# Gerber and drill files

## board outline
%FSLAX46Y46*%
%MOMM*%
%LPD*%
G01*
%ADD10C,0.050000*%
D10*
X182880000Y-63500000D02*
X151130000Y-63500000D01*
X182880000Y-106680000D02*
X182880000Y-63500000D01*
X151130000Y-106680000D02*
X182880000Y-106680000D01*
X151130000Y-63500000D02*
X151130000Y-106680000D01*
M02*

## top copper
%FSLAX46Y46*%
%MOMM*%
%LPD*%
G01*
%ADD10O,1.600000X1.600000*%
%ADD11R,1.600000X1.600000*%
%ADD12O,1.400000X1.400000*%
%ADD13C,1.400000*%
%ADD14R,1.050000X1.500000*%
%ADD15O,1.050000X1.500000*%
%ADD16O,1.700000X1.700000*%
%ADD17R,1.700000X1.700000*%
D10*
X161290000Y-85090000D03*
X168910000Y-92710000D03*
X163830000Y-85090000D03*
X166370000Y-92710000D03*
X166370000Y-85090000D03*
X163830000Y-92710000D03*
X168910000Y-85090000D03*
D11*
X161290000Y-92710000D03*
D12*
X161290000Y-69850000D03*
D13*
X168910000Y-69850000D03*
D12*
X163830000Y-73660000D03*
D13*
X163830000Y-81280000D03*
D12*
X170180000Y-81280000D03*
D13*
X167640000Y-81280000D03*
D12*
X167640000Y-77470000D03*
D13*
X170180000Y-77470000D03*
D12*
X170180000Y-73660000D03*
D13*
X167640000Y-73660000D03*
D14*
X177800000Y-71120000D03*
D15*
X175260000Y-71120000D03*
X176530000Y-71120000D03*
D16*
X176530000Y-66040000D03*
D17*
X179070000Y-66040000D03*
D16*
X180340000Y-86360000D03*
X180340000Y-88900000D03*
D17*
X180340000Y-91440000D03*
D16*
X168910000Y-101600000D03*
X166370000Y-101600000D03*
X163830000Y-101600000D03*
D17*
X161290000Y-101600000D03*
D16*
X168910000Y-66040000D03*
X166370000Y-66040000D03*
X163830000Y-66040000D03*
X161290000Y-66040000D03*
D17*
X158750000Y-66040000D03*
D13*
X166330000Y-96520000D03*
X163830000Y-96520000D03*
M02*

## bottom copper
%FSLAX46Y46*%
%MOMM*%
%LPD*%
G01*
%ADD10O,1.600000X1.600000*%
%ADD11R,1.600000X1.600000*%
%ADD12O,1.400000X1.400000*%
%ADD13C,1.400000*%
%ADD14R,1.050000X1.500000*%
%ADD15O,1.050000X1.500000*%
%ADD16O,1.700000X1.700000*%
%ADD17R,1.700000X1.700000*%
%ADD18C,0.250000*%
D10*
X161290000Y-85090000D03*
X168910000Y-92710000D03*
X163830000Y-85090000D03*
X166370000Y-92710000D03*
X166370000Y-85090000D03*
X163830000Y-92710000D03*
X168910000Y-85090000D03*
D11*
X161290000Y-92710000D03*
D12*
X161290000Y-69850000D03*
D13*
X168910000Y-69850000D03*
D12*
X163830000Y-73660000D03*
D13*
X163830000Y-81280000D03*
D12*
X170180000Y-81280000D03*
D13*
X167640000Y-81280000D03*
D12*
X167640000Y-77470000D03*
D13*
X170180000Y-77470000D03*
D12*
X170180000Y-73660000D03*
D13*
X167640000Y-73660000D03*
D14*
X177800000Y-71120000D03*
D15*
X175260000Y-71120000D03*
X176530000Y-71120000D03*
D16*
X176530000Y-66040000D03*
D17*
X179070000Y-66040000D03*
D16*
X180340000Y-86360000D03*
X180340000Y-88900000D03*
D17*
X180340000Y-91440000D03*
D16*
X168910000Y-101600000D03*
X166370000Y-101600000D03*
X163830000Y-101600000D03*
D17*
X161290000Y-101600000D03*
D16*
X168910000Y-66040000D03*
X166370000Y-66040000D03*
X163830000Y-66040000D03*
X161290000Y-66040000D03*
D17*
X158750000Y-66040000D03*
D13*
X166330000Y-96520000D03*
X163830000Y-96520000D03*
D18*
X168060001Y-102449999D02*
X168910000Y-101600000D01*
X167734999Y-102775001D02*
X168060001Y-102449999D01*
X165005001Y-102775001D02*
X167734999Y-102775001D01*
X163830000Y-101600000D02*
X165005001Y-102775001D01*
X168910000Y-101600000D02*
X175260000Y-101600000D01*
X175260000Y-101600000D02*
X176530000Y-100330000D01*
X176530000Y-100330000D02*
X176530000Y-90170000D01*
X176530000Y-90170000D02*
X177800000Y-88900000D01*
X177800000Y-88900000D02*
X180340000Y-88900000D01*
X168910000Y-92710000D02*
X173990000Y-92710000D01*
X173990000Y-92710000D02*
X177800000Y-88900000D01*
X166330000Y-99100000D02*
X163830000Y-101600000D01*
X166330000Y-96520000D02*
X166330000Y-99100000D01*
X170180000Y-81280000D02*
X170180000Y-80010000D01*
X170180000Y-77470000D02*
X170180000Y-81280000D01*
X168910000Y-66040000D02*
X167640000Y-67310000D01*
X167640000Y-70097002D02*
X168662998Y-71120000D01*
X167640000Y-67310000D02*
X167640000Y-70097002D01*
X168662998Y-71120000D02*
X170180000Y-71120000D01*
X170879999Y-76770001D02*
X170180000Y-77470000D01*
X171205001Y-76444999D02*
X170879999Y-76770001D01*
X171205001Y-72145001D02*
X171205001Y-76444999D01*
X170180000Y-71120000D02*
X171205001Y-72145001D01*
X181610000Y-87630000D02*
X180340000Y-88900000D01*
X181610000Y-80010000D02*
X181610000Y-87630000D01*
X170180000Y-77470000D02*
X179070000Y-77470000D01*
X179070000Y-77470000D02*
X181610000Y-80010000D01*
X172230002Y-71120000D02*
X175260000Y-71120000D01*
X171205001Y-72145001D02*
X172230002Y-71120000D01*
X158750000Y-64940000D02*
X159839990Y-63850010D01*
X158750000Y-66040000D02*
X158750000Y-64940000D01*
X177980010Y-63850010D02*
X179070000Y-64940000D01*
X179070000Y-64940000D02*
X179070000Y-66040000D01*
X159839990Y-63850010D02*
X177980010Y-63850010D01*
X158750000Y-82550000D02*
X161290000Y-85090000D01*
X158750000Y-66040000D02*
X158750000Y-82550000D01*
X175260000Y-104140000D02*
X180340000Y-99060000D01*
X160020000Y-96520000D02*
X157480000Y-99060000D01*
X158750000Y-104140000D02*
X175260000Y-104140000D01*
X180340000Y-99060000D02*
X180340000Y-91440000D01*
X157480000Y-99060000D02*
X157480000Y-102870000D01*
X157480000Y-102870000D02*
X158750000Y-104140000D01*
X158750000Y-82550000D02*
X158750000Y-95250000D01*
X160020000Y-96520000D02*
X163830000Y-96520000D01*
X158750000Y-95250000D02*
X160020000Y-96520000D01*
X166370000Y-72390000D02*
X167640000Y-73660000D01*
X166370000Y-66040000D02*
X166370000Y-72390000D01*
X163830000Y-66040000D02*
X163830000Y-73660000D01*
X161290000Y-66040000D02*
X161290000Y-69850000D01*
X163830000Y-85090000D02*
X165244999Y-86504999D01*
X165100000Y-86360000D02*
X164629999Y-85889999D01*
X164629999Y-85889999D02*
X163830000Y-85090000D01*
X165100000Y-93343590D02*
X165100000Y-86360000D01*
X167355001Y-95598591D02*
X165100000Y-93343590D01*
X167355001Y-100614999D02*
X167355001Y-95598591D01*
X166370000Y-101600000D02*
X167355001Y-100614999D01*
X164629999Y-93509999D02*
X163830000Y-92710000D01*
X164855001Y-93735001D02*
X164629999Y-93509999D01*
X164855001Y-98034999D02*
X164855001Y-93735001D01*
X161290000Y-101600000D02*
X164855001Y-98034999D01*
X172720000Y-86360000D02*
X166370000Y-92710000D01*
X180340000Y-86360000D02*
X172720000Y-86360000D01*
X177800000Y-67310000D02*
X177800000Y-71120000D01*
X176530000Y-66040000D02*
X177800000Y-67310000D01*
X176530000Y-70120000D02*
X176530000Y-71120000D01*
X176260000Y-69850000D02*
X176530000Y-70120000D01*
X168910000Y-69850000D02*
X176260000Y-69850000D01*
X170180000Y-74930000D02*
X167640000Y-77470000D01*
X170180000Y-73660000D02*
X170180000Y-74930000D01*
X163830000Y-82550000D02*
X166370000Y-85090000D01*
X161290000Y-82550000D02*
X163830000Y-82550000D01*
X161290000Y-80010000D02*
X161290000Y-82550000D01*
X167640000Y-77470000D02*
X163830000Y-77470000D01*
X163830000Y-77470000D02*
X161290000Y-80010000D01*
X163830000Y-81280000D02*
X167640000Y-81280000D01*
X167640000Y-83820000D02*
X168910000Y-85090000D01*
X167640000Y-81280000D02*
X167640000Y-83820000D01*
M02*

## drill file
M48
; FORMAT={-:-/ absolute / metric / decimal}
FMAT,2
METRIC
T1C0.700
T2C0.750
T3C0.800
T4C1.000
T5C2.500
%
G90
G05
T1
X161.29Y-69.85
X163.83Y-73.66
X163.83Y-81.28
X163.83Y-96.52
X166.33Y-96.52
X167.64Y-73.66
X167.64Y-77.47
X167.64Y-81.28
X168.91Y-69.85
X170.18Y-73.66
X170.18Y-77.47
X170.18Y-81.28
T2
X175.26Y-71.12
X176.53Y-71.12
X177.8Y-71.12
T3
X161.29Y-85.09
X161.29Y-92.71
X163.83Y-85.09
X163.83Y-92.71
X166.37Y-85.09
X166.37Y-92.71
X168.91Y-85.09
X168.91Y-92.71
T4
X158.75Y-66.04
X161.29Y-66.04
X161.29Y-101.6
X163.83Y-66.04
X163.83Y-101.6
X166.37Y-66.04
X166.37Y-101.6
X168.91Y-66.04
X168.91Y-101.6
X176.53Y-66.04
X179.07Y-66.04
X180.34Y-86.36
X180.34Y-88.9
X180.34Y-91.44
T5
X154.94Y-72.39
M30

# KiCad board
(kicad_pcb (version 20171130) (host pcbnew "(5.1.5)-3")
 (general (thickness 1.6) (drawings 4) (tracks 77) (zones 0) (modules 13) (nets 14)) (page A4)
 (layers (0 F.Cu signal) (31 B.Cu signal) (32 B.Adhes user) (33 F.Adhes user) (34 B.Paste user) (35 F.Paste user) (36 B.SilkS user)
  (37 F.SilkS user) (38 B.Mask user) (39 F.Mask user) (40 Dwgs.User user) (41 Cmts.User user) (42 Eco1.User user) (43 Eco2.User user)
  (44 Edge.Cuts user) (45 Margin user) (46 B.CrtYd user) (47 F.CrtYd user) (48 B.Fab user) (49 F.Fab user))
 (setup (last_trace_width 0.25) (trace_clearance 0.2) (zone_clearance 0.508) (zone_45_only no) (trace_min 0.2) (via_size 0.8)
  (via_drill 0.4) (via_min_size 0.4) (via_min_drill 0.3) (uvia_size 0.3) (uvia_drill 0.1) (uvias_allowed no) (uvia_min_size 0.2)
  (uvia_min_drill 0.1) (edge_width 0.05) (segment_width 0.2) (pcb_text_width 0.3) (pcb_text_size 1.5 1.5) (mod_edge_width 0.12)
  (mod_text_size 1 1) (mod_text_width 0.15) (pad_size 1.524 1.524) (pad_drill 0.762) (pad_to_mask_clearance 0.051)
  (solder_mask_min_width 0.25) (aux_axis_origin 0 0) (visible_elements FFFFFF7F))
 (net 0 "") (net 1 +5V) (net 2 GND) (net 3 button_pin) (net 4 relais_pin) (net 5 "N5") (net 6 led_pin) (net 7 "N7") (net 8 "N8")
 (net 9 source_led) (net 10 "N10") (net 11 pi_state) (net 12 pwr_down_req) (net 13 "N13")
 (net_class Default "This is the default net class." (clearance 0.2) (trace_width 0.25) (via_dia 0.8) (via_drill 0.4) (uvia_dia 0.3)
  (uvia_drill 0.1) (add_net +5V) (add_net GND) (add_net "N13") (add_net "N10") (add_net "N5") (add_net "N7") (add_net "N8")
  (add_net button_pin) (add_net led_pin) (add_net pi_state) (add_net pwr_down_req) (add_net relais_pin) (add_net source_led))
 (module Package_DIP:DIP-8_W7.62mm (layer F.Cu) (at 161.29 92.71 90)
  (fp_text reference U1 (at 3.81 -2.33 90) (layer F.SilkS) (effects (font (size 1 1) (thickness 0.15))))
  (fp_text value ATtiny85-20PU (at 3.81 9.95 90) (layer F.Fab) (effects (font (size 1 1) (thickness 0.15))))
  (pad 8 thru_hole oval (at 7.62 0 90) (size 1.6 1.6) (drill 0.8) (layers *.Cu *.Mask) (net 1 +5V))
  (pad 4 thru_hole oval (at 0 7.62 90) (size 1.6 1.6) (drill 0.8) (layers *.Cu *.Mask) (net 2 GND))
  (pad 7 thru_hole oval (at 7.62 2.54 90) (size 1.6 1.6) (drill 0.8) (layers *.Cu *.Mask) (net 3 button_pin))
  (pad 3 thru_hole oval (at 0 5.08 90) (size 1.6 1.6) (drill 0.8) (layers *.Cu *.Mask) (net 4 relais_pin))
  (pad 6 thru_hole oval (at 7.62 5.08 90) (size 1.6 1.6) (drill 0.8) (layers *.Cu *.Mask) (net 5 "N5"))
  (pad 2 thru_hole oval (at 0 2.54 90) (size 1.6 1.6) (drill 0.8) (layers *.Cu *.Mask) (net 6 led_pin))
  (pad 5 thru_hole oval (at 7.62 7.62 90) (size 1.6 1.6) (drill 0.8) (layers *.Cu *.Mask) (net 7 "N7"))
  (pad 1 thru_hole rect (at 0 0 90) (size 1.6 1.6) (drill 0.8) (layers *.Cu *.Mask) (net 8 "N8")))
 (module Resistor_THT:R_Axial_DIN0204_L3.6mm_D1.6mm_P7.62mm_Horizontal (layer F.Cu) (at 168.91 69.85 180)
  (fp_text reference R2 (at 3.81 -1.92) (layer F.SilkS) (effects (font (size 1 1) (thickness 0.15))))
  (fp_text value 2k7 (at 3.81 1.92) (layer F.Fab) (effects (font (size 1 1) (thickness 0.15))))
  (pad 2 thru_hole oval (at 7.62 0 180) (size 1.4 1.4) (drill 0.7) (layers *.Cu *.Mask) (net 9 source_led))
  (pad 1 thru_hole circle (at 0 0 180) (size 1.4 1.4) (drill 0.7) (layers *.Cu *.Mask) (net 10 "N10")))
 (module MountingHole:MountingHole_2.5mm (layer F.Cu) (at 154.94 72.39)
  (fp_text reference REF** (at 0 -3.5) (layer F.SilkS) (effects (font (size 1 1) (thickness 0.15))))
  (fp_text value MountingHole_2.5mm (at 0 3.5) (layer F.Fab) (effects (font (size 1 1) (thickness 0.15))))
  (pad 1 np_thru_hole circle (at 0 0) (size 2.5 2.5) (drill 2.5) (layers *.Cu *.Mask)))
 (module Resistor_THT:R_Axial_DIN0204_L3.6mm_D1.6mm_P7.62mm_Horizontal (layer F.Cu) (at 163.83 81.28 90)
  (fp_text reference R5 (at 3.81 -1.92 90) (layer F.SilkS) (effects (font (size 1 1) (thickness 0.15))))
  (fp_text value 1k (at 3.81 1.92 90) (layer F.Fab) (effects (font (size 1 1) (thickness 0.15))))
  (pad 2 thru_hole oval (at 7.62 0 90) (size 1.4 1.4) (drill 0.7) (layers *.Cu *.Mask) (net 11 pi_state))
  (pad 1 thru_hole circle (at 0 0 90) (size 1.4 1.4) (drill 0.7) (layers *.Cu *.Mask) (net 7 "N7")))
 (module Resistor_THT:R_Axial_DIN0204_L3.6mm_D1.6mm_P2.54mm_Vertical (layer F.Cu) (at 167.64 81.28)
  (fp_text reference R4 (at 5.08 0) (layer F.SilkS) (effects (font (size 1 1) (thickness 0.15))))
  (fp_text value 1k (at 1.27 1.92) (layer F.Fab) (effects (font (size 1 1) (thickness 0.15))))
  (pad 2 thru_hole oval (at 2.54 0) (size 1.4 1.4) (drill 0.7) (layers *.Cu *.Mask) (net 2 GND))
  (pad 1 thru_hole circle (at 0 0) (size 1.4 1.4) (drill 0.7) (layers *.Cu *.Mask) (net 7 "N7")))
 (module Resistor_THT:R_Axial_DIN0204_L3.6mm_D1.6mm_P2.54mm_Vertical (layer F.Cu) (at 170.18 77.47 180)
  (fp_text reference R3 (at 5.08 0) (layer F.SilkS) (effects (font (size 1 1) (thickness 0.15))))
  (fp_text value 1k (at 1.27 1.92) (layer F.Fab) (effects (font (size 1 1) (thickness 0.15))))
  (pad 2 thru_hole oval (at 2.54 0 180) (size 1.4 1.4) (drill 0.7) (layers *.Cu *.Mask) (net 5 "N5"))
  (pad 1 thru_hole circle (at 0 0 180) (size 1.4 1.4) (drill 0.7) (layers *.Cu *.Mask) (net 2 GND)))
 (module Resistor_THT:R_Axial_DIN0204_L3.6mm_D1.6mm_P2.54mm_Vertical (layer F.Cu) (at 167.64 73.66)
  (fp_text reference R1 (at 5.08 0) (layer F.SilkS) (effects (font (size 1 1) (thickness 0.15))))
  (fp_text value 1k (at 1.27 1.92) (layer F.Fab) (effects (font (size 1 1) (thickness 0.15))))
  (pad 2 thru_hole oval (at 2.54 0) (size 1.4 1.4) (drill 0.7) (layers *.Cu *.Mask) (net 5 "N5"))
  (pad 1 thru_hole circle (at 0 0) (size 1.4 1.4) (drill 0.7) (layers *.Cu *.Mask) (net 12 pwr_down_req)))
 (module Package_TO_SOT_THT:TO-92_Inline (layer F.Cu) (at 177.8 71.12 180)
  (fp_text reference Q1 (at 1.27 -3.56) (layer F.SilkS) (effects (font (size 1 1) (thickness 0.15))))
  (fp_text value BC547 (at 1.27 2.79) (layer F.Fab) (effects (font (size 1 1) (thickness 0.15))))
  (pad 1 thru_hole rect (at 0 0 180) (size 1.05 1.5) (drill 0.75) (layers *.Cu *.Mask) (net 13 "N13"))
  (pad 3 thru_hole oval (at 2.54 0 180) (size 1.05 1.5) (drill 0.75) (layers *.Cu *.Mask) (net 2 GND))
  (pad 2 thru_hole oval (at 1.27 0 180) (size 1.05 1.5) (drill 0.75) (layers *.Cu *.Mask) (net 10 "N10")))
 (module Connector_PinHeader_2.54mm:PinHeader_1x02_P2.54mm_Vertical (layer F.Cu) (at 179.07 66.04 270)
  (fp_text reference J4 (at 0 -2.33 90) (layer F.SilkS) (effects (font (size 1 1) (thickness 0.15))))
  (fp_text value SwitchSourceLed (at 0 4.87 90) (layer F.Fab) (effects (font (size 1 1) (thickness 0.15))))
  (pad 2 thru_hole oval (at 0 2.54 270) (size 1.7 1.7) (drill 1) (layers *.Cu *.Mask) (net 13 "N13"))
  (pad 1 thru_hole rect (at 0 0 270) (size 1.7 1.7) (drill 1) (layers *.Cu *.Mask) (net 1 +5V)))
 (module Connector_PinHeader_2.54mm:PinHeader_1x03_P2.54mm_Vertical (layer F.Cu) (at 180.34 91.44 180)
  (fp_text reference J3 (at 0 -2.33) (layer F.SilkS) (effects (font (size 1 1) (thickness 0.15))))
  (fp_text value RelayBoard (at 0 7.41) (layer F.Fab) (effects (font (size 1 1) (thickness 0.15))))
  (pad 3 thru_hole oval (at 0 5.08 180) (size 1.7 1.7) (drill 1) (layers *.Cu *.Mask) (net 4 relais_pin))
  (pad 2 thru_hole oval (at 0 2.54 180) (size 1.7 1.7) (drill 1) (layers *.Cu *.Mask) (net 2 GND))
  (pad 1 thru_hole rect (at 0 0 180) (size 1.7 1.7) (drill 1) (layers *.Cu *.Mask) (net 1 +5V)))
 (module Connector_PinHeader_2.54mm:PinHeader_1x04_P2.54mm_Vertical (layer F.Cu) (at 161.29 101.6 90)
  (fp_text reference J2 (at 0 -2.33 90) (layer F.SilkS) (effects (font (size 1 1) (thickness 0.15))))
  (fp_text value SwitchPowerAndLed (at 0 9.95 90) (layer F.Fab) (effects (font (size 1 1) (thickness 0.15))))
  (pad 4 thru_hole oval (at 0 7.62 90) (size 1.7 1.7) (drill 1) (layers *.Cu *.Mask) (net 2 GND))
  (pad 3 thru_hole oval (at 0 5.08 90) (size 1.7 1.7) (drill 1) (layers *.Cu *.Mask) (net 3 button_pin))
  (pad 2 thru_hole oval (at 0 2.54 90) (size 1.7 1.7) (drill 1) (layers *.Cu *.Mask) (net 2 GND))
  (pad 1 thru_hole rect (at 0 0 90) (size 1.7 1.7) (drill 1) (layers *.Cu *.Mask) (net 6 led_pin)))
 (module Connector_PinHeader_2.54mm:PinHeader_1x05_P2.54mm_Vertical (layer F.Cu) (at 158.75 66.04 90)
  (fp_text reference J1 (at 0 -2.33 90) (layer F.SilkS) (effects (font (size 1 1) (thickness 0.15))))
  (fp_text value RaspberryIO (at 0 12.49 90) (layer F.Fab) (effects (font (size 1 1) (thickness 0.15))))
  (pad 5 thru_hole oval (at 0 10.16 90) (size 1.7 1.7) (drill 1) (layers *.Cu *.Mask) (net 2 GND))
  (pad 4 thru_hole oval (at 0 7.62 90) (size 1.7 1.7) (drill 1) (layers *.Cu *.Mask) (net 12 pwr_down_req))
  (pad 3 thru_hole oval (at 0 5.08 90) (size 1.7 1.7) (drill 1) (layers *.Cu *.Mask) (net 11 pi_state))
  (pad 2 thru_hole oval (at 0 2.54 90) (size 1.7 1.7) (drill 1) (layers *.Cu *.Mask) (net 9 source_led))
  (pad 1 thru_hole rect (at 0 0 90) (size 1.7 1.7) (drill 1) (layers *.Cu *.Mask) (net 1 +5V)))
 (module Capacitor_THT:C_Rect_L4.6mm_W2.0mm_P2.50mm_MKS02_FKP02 (layer F.Cu) (at 163.83 96.52)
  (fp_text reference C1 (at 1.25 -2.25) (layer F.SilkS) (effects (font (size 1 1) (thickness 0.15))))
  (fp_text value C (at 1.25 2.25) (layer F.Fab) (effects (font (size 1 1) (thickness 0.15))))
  (pad 2 thru_hole circle (at 2.5 0) (size 1.4 1.4) (drill 0.7) (layers *.Cu *.Mask) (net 2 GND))
  (pad 1 thru_hole circle (at 0 0) (size 1.4 1.4) (drill 0.7) (layers *.Cu *.Mask) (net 1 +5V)))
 (gr_line (start 182.88 63.5) (end 151.13 63.5) (layer Edge.Cuts) (width 0.05))
 (gr_line (start 182.88 106.68) (end 182.88 63.5) (layer Edge.Cuts) (width 0.05))
 (gr_line (start 151.13 106.68) (end 182.88 106.68) (layer Edge.Cuts) (width 0.05))
 (gr_line (start 151.13 63.5) (end 151.13 106.68) (layer Edge.Cuts) (width 0.05))
 (segment (start 168.060001 102.449999) (end 168.91 101.6) (width 0.25) (layer B.Cu) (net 2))
 (segment (start 167.734999 102.775001) (end 168.060001 102.449999) (width 0.25) (layer B.Cu) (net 2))
 (segment (start 165.005001 102.775001) (end 167.734999 102.775001) (width 0.25) (layer B.Cu) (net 2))
 (segment (start 163.83 101.6) (end 165.005001 102.775001) (width 0.25) (layer B.Cu) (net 2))
 (segment (start 168.91 101.6) (end 175.26 101.6) (width 0.25) (layer B.Cu) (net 2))
 (segment (start 175.26 101.6) (end 176.53 100.33) (width 0.25) (layer B.Cu) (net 2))
 (segment (start 176.53 100.33) (end 176.53 90.17) (width 0.25) (layer B.Cu) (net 2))
 (segment (start 176.53 90.17) (end 177.8 88.9) (width 0.25) (layer B.Cu) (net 2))
 (segment (start 177.8 88.9) (end 180.34 88.9) (width 0.25) (layer B.Cu) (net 2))
 (segment (start 168.91 92.71) (end 173.99 92.71) (width 0.25) (layer B.Cu) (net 2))
 (segment (start 173.99 92.71) (end 177.8 88.9) (width 0.25) (layer B.Cu) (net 2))
 (segment (start 166.33 99.1) (end 163.83 101.6) (width 0.25) (layer B.Cu) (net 2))
 (segment (start 166.33 96.52) (end 166.33 99.1) (width 0.25) (layer B.Cu) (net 2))
 (segment (start 170.18 81.28) (end 170.18 80.01) (width 0.25) (layer B.Cu) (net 2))
 (segment (start 170.18 77.47) (end 170.18 81.28) (width 0.25) (layer B.Cu) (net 2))
 (segment (start 168.91 66.04) (end 167.64 67.31) (width 0.25) (layer B.Cu) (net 2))
 (segment (start 167.64 70.097002) (end 168.662998 71.12) (width 0.25) (layer B.Cu) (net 2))
 (segment (start 167.64 67.31) (end 167.64 70.097002) (width 0.25) (layer B.Cu) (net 2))
 (segment (start 168.662998 71.12) (end 170.18 71.12) (width 0.25) (layer B.Cu) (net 2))
 (segment (start 170.879999 76.770001) (end 170.18 77.47) (width 0.25) (layer B.Cu) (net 2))
 (segment (start 171.205001 76.444999) (end 170.879999 76.770001) (width 0.25) (layer B.Cu) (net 2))
 (segment (start 171.205001 72.145001) (end 171.205001 76.444999) (width 0.25) (layer B.Cu) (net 2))
 (segment (start 170.18 71.12) (end 171.205001 72.145001) (width 0.25) (layer B.Cu) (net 2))
 (segment (start 181.61 87.63) (end 180.34 88.9) (width 0.25) (layer B.Cu) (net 2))
 (segment (start 181.61 80.01) (end 181.61 87.63) (width 0.25) (layer B.Cu) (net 2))
 (segment (start 170.18 77.47) (end 179.07 77.47) (width 0.25) (layer B.Cu) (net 2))
 (segment (start 179.07 77.47) (end 181.61 80.01) (width 0.25) (layer B.Cu) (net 2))
 (segment (start 172.230002 71.12) (end 175.26 71.12) (width 0.25) (layer B.Cu) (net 2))
 (segment (start 171.205001 72.145001) (end 172.230002 71.12) (width 0.25) (layer B.Cu) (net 2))
 (segment (start 158.75 64.94) (end 159.83999 63.85001) (width 0.25) (layer B.Cu) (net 1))
 (segment (start 158.75 66.04) (end 158.75 64.94) (width 0.25) (layer B.Cu) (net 1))
 (segment (start 177.98001 63.85001) (end 179.07 64.94) (width 0.25) (layer B.Cu) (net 1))
 (segment (start 179.07 64.94) (end 179.07 66.04) (width 0.25) (layer B.Cu) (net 1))
 (segment (start 159.83999 63.85001) (end 177.98001 63.85001) (width 0.25) (layer B.Cu) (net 1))
 (segment (start 158.75 82.55) (end 161.29 85.09) (width 0.25) (layer B.Cu) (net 1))
 (segment (start 158.75 66.04) (end 158.75 82.55) (width 0.25) (layer B.Cu) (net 1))
 (segment (start 175.26 104.14) (end 180.34 99.06) (width 0.25) (layer B.Cu) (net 1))
 (segment (start 160.02 96.52) (end 157.48 99.06) (width 0.25) (layer B.Cu) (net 1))
 (segment (start 158.75 104.14) (end 175.26 104.14) (width 0.25) (layer B.Cu) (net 1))
 (segment (start 180.34 99.06) (end 180.34 91.44) (width 0.25) (layer B.Cu) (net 1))
 (segment (start 157.48 99.06) (end 157.48 102.87) (width 0.25) (layer B.Cu) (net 1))
 (segment (start 157.48 102.87) (end 158.75 104.14) (width 0.25) (layer B.Cu) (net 1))
 (segment (start 158.75 82.55) (end 158.75 95.25) (width 0.25) (layer B.Cu) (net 1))
 (segment (start 160.02 96.52) (end 163.83 96.52) (width 0.25) (layer B.Cu) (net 1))
 (segment (start 158.75 95.25) (end 160.02 96.52) (width 0.25) (layer B.Cu) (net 1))
 (segment (start 166.37 72.39) (end 167.64 73.66) (width 0.25) (layer B.Cu) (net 12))
 (segment (start 166.37 66.04) (end 166.37 72.39) (width 0.25) (layer B.Cu) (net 12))
 (segment (start 163.83 66.04) (end 163.83 73.66) (width 0.25) (layer B.Cu) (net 11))
 (segment (start 161.29 66.04) (end 161.29 69.85) (width 0.25) (layer B.Cu) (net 9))
 (segment (start 163.83 85.09) (end 165.244999 86.504999) (width 0.25) (layer B.Cu) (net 3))
 (segment (start 165.1 86.36) (end 164.629999 85.889999) (width 0.25) (layer B.Cu) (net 3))
 (segment (start 164.629999 85.889999) (end 163.83 85.09) (width 0.25) (layer B.Cu) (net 3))
 (segment (start 165.1 93.34359) (end 165.1 86.36) (width 0.25) (layer B.Cu) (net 3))
 (segment (start 167.355001 95.598591) (end 165.1 93.34359) (width 0.25) (layer B.Cu) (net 3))
 (segment (start 167.355001 100.614999) (end 167.355001 95.598591) (width 0.25) (layer B.Cu) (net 3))
 (segment (start 166.37 101.6) (end 167.355001 100.614999) (width 0.25) (layer B.Cu) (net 3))
 (segment (start 164.629999 93.509999) (end 163.83 92.71) (width 0.25) (layer B.Cu) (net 6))
 (segment (start 164.855001 93.735001) (end 164.629999 93.509999) (width 0.25) (layer B.Cu) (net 6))
 (segment (start 164.855001 98.034999) (end 164.855001 93.735001) (width 0.25) (layer B.Cu) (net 6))
 (segment (start 161.29 101.6) (end 164.855001 98.034999) (width 0.25) (layer B.Cu) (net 6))
 (segment (start 172.72 86.36) (end 166.37 92.71) (width 0.25) (layer B.Cu) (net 4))
 (segment (start 180.34 86.36) (end 172.72 86.36) (width 0.25) (layer B.Cu) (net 4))
 (segment (start 177.8 67.31) (end 177.8 71.12) (width 0.25) (layer B.Cu) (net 13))
 (segment (start 176.53 66.04) (end 177.8 67.31) (width 0.25) (layer B.Cu) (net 13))
 (segment (start 176.53 70.12) (end 176.53 71.12) (width 0.25) (layer B.Cu) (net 10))
 (segment (start 176.26 69.85) (end 176.53 70.12) (width 0.25) (layer B.Cu) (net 10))
 (segment (start 168.91 69.85) (end 176.26 69.85) (width 0.25) (layer B.Cu) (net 10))
 (segment (start 170.18 74.93) (end 167.64 77.47) (width 0.25) (layer B.Cu) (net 5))
 (segment (start 170.18 73.66) (end 170.18 74.93) (width 0.25) (layer B.Cu) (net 5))
 (segment (start 163.83 82.55) (end 166.37 85.09) (width 0.25) (layer B.Cu) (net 5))
 (segment (start 161.29 82.55) (end 163.83 82.55) (width 0.25) (layer B.Cu) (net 5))
 (segment (start 161.29 80.01) (end 161.29 82.55) (width 0.25) (layer B.Cu) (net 5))
 (segment (start 167.64 77.47) (end 163.83 77.47) (width 0.25) (layer B.Cu) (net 5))
 (segment (start 163.83 77.47) (end 161.29 80.01) (width 0.25) (layer B.Cu) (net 5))
 (segment (start 163.83 81.28) (end 167.64 81.28) (width 0.25) (layer B.Cu) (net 7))
 (segment (start 167.64 83.82) (end 168.91 85.09) (width 0.25) (layer B.Cu) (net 7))
 (segment (start 167.64 81.28) (end 167.64 83.82) (width 0.25) (layer B.Cu) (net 7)))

